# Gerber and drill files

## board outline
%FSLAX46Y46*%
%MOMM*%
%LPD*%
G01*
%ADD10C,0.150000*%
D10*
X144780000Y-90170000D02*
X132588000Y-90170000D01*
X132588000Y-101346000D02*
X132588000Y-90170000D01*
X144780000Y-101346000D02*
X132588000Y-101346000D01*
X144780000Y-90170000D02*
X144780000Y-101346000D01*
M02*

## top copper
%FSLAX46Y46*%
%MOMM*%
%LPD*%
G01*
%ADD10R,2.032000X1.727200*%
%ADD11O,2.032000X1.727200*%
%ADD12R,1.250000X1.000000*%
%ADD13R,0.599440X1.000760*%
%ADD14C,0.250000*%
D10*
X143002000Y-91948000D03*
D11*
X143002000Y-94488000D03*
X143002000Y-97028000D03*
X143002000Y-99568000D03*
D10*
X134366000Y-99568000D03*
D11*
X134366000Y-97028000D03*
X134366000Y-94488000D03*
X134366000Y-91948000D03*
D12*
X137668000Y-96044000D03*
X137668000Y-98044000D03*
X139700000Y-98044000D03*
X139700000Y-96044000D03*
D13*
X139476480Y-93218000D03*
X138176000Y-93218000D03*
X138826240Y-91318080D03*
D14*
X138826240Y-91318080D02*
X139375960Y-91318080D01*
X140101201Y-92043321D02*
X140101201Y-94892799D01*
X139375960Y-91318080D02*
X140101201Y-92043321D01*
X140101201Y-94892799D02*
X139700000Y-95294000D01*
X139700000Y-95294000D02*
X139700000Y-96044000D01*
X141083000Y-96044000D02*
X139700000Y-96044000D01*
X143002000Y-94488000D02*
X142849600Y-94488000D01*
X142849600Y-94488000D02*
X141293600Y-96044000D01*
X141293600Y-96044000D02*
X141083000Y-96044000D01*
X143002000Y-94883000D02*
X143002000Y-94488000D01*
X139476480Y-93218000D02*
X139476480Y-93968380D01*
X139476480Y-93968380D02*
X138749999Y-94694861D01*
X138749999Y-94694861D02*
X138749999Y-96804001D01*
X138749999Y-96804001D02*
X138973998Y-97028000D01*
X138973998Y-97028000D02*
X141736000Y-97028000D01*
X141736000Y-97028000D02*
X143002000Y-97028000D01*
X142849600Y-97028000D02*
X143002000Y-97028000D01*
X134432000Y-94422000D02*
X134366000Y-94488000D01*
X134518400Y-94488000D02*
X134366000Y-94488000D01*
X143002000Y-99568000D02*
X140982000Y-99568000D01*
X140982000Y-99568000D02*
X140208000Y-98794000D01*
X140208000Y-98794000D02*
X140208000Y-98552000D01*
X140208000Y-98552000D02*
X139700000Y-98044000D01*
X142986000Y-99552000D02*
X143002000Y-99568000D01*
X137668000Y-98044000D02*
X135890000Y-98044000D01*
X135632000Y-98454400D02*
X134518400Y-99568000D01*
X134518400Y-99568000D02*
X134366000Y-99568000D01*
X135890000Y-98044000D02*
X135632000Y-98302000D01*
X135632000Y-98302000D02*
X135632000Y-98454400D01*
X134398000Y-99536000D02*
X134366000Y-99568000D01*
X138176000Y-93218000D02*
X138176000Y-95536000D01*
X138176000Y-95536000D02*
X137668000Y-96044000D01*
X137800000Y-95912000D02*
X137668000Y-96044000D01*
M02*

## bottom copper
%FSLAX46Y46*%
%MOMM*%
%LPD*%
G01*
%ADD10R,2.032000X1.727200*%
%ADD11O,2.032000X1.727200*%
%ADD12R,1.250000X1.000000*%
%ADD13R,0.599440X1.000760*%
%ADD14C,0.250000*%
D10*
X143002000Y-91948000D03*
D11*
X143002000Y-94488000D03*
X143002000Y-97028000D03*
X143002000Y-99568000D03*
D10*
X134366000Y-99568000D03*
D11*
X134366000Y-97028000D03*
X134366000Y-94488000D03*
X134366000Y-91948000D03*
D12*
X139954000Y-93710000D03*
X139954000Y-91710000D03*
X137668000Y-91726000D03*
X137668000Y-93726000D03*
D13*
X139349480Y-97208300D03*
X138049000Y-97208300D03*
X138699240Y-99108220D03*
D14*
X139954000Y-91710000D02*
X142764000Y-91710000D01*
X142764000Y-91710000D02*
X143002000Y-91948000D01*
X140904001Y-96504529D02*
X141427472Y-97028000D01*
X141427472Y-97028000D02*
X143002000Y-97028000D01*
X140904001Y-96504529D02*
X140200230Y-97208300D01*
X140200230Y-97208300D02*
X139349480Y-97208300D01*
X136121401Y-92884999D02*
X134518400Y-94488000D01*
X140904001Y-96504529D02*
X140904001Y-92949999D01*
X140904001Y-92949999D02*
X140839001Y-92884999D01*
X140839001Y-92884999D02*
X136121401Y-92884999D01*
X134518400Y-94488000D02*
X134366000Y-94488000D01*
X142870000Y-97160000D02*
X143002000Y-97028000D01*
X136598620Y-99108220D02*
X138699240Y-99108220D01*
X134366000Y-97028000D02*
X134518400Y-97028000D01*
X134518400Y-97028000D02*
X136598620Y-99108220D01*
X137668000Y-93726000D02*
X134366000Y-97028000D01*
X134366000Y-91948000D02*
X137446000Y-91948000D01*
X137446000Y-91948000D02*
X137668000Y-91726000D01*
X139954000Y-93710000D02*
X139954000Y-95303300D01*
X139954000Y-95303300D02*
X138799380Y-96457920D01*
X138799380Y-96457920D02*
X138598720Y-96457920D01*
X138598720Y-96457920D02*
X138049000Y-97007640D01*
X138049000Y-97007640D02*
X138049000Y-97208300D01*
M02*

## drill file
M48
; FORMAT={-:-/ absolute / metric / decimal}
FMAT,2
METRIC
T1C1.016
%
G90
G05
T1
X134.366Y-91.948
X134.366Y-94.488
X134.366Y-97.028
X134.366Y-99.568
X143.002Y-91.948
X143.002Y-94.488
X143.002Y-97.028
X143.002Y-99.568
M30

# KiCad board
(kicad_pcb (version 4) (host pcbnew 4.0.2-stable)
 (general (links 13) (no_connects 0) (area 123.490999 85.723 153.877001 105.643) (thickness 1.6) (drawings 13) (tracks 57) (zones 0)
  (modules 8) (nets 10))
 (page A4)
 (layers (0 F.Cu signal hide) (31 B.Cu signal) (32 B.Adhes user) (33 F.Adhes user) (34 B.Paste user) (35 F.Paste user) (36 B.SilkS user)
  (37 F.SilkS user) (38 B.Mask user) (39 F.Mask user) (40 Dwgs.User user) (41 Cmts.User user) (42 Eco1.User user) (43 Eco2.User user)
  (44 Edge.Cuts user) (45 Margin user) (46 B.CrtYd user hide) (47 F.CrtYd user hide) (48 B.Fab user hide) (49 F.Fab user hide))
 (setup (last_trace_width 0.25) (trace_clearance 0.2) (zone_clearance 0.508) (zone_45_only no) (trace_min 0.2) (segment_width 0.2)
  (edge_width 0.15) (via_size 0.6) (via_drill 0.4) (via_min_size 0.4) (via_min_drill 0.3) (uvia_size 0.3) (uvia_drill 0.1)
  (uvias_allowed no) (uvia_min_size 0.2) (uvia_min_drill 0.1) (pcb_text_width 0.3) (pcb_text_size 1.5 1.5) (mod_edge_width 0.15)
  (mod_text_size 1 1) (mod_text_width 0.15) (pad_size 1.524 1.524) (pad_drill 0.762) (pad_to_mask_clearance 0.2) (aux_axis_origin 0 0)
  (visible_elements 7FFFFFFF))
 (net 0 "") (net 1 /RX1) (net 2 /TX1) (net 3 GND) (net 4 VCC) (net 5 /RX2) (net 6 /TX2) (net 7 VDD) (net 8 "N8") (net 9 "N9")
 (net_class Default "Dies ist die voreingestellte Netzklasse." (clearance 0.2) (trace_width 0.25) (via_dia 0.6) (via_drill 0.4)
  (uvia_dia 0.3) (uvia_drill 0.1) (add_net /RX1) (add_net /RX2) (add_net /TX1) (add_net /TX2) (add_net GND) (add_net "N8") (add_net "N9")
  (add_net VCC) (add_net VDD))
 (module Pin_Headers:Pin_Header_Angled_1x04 (layer F.Cu) (at 143.002 91.948)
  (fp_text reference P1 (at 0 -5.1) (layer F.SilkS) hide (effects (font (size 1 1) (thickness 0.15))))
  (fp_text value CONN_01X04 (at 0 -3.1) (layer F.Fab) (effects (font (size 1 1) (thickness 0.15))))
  (pad 1 thru_hole rect (at 0 0) (size 2.032 1.7272) (drill 1.016) (layers *.Cu *.Mask F.SilkS) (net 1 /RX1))
  (pad 2 thru_hole oval (at 0 2.54) (size 2.032 1.7272) (drill 1.016) (layers *.Cu *.Mask F.SilkS) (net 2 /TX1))
  (pad 3 thru_hole oval (at 0 5.08) (size 2.032 1.7272) (drill 1.016) (layers *.Cu *.Mask F.SilkS) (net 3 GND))
  (pad 4 thru_hole oval (at 0 7.62) (size 2.032 1.7272) (drill 1.016) (layers *.Cu *.Mask F.SilkS) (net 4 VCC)))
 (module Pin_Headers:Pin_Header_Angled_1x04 (layer F.Cu) (at 134.366 99.568 180)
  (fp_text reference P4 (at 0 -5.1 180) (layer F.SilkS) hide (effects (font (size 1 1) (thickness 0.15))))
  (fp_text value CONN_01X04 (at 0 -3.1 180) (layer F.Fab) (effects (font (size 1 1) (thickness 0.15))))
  (pad 1 thru_hole rect (at 0 0 180) (size 2.032 1.7272) (drill 1.016) (layers *.Cu *.Mask F.SilkS) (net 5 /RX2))
  (pad 2 thru_hole oval (at 0 2.54 180) (size 2.032 1.7272) (drill 1.016) (layers *.Cu *.Mask F.SilkS) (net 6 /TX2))
  (pad 3 thru_hole oval (at 0 5.08 180) (size 2.032 1.7272) (drill 1.016) (layers *.Cu *.Mask F.SilkS) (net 3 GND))
  (pad 4 thru_hole oval (at 0 7.62 180) (size 2.032 1.7272) (drill 1.016) (layers *.Cu *.Mask F.SilkS) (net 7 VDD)))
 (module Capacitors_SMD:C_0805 (layer B.Cu) (at 139.954 92.71 90)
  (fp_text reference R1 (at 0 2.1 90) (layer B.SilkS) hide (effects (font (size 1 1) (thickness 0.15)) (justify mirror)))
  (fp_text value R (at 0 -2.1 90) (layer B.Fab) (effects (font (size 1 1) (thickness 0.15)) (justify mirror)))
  (pad 1 smd rect (at -1 0 90) (size 1 1.25) (layers B.Cu B.Paste B.Mask) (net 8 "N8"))
  (pad 2 smd rect (at 1 0 90) (size 1 1.25) (layers B.Cu B.Paste B.Mask) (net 1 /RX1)))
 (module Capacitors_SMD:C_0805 (layer F.Cu) (at 137.668 97.044 270)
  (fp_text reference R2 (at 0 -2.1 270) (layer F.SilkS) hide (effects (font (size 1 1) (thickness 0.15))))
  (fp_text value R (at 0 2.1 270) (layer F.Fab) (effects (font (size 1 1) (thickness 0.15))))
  (pad 1 smd rect (at -1 0 270) (size 1 1.25) (layers F.Cu F.Paste F.Mask) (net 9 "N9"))
  (pad 2 smd rect (at 1 0 270) (size 1 1.25) (layers F.Cu F.Paste F.Mask) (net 5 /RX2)))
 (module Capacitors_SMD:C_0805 (layer B.Cu) (at 137.668 92.726 270)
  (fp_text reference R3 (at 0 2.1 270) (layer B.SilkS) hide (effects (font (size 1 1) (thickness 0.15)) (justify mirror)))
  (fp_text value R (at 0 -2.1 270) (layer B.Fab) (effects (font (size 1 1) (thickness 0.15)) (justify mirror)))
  (pad 1 smd rect (at -1 0 270) (size 1 1.25) (layers B.Cu B.Paste B.Mask) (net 7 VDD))
  (pad 2 smd rect (at 1 0 270) (size 1 1.25) (layers B.Cu B.Paste B.Mask) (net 6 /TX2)))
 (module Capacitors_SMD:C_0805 (layer F.Cu) (at 139.7 97.044 90)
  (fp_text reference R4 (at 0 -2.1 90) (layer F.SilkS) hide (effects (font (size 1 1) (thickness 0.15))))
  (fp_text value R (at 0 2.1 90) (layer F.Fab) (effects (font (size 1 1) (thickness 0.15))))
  (pad 1 smd rect (at -1 0 90) (size 1 1.25) (layers F.Cu F.Paste F.Mask) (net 4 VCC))
  (pad 2 smd rect (at 1 0 90) (size 1 1.25) (layers F.Cu F.Paste F.Mask) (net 2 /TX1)))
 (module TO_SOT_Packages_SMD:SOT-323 (layer B.Cu) (at 138.69924 98.15826 180)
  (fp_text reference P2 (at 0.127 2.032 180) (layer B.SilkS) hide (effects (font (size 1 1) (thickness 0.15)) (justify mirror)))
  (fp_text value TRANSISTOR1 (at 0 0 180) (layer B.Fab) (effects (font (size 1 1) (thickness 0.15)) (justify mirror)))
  (pad 2 smd rect (at -0.65024 0.94996 180) (size 0.59944 1.00076) (layers B.Cu B.Paste B.Mask) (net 3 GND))
  (pad 1 smd rect (at 0.65024 0.94996 180) (size 0.59944 1.00076) (layers B.Cu B.Paste B.Mask) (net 8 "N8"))
  (pad 3 smd rect (at 0 -0.94996 180) (size 0.59944 1.00076) (layers B.Cu B.Paste B.Mask) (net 6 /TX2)))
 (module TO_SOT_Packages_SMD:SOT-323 (layer F.Cu) (at 138.82624 92.26804 180)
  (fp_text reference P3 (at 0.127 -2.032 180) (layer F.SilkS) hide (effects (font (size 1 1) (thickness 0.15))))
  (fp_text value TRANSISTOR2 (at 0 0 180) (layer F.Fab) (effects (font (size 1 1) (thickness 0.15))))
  (pad 2 smd rect (at -0.65024 -0.94996 180) (size 0.59944 1.00076) (layers F.Cu F.Paste F.Mask) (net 3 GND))
  (pad 1 smd rect (at 0.65024 -0.94996 180) (size 0.59944 1.00076) (layers F.Cu F.Paste F.Mask) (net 9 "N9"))
  (pad 3 smd rect (at 0 0.94996 180) (size 0.59944 1.00076) (layers F.Cu F.Paste F.Mask) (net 2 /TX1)))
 (gr_line (start 144.78 90.17) (end 132.588 90.17) (layer Edge.Cuts) (width 0.15))
 (gr_line (start 132.588 101.346) (end 132.588 90.17) (layer Edge.Cuts) (width 0.15))
 (gr_line (start 144.78 101.346) (end 132.588 101.346) (layer Edge.Cuts) (width 0.15))
 (gr_line (start 144.78 90.17) (end 144.78 101.346) (layer Edge.Cuts) (width 0.15))
 (segment (start 144.78 90.17) (end 132.588 90.17) (width 0.25) (layer Dwgs.User) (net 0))
 (segment (start 139.954 91.71) (end 142.764 91.71) (width 0.25) (layer B.Cu) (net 1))
 (segment (start 142.764 91.71) (end 143.002 91.948) (width 0.25) (layer B.Cu) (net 1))
 (segment (start 138.82624 91.31808) (end 139.37596 91.31808) (width 0.25) (layer F.Cu) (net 2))
 (segment (start 140.101201 92.043321) (end 140.101201 94.892799) (width 0.25) (layer F.Cu) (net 2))
 (segment (start 139.37596 91.31808) (end 140.101201 92.043321) (width 0.25) (layer F.Cu) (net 2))
 (segment (start 140.101201 94.892799) (end 139.7 95.294) (width 0.25) (layer F.Cu) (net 2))
 (segment (start 139.7 95.294) (end 139.7 96.044) (width 0.25) (layer F.Cu) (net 2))
 (segment (start 141.083 96.044) (end 139.7 96.044) (width 0.25) (layer F.Cu) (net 2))
 (segment (start 143.002 94.488) (end 142.8496 94.488) (width 0.25) (layer F.Cu) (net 2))
 (segment (start 142.8496 94.488) (end 141.2936 96.044) (width 0.25) (layer F.Cu) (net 2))
 (segment (start 141.2936 96.044) (end 141.083 96.044) (width 0.25) (layer F.Cu) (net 2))
 (segment (start 143.002 94.883) (end 143.002 94.488) (width 0.25) (layer F.Cu) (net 2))
 (segment (start 140.904001 96.504529) (end 141.427472 97.028) (width 0.25) (layer B.Cu) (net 3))
 (segment (start 141.427472 97.028) (end 143.002 97.028) (width 0.25) (layer B.Cu) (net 3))
 (segment (start 140.904001 96.504529) (end 140.20023 97.2083) (width 0.25) (layer B.Cu) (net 3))
 (segment (start 140.20023 97.2083) (end 139.34948 97.2083) (width 0.25) (layer B.Cu) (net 3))
 (segment (start 139.47648 93.218) (end 139.47648 93.96838) (width 0.25) (layer F.Cu) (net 3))
 (segment (start 139.47648 93.96838) (end 138.749999 94.694861) (width 0.25) (layer F.Cu) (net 3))
 (segment (start 138.749999 94.694861) (end 138.749999 96.804001) (width 0.25) (layer F.Cu) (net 3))
 (segment (start 138.749999 96.804001) (end 138.973998 97.028) (width 0.25) (layer F.Cu) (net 3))
 (segment (start 138.973998 97.028) (end 141.736 97.028) (width 0.25) (layer F.Cu) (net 3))
 (segment (start 141.736 97.028) (end 143.002 97.028) (width 0.25) (layer F.Cu) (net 3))
 (segment (start 136.121401 92.884999) (end 134.5184 94.488) (width 0.25) (layer B.Cu) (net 3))
 (segment (start 140.904001 96.504529) (end 140.904001 92.949999) (width 0.25) (layer B.Cu) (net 3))
 (segment (start 140.904001 92.949999) (end 140.839001 92.884999) (width 0.25) (layer B.Cu) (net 3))
 (segment (start 140.839001 92.884999) (end 136.121401 92.884999) (width 0.25) (layer B.Cu) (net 3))
 (segment (start 134.5184 94.488) (end 134.366 94.488) (width 0.25) (layer B.Cu) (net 3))
 (segment (start 142.8496 97.028) (end 143.002 97.028) (width 0.25) (layer F.Cu) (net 3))
 (segment (start 134.432 94.422) (end 134.366 94.488) (width 0.25) (layer F.Cu) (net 3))
 (segment (start 142.87 97.16) (end 143.002 97.028) (width 0.25) (layer B.Cu) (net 3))
 (segment (start 134.5184 94.488) (end 134.366 94.488) (width 0.25) (layer F.Cu) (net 3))
 (segment (start 143.002 99.568) (end 140.982 99.568) (width 0.25) (layer F.Cu) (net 4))
 (segment (start 140.982 99.568) (end 140.208 98.794) (width 0.25) (layer F.Cu) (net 4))
 (segment (start 140.208 98.794) (end 140.208 98.552) (width 0.25) (layer F.Cu) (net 4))
 (segment (start 140.208 98.552) (end 139.7 98.044) (width 0.25) (layer F.Cu) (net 4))
 (segment (start 142.986 99.552) (end 143.002 99.568) (width 0.25) (layer F.Cu) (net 4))
 (segment (start 136.59862 99.10822) (end 138.69924 99.10822) (width 0.25) (layer B.Cu) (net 6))
 (segment (start 134.366 97.028) (end 134.5184 97.028) (width 0.25) (layer B.Cu) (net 6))
 (segment (start 134.5184 97.028) (end 136.59862 99.10822) (width 0.25) (layer B.Cu) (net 6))
 (segment (start 137.668 93.726) (end 134.366 97.028) (width 0.25) (layer B.Cu) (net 6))
 (segment (start 137.668 98.044) (end 135.89 98.044) (width 0.25) (layer F.Cu) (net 5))
 (segment (start 135.632 98.4544) (end 134.5184 99.568) (width 0.25) (layer F.Cu) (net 5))
 (segment (start 134.5184 99.568) (end 134.366 99.568) (width 0.25) (layer F.Cu) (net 5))
 (segment (start 135.89 98.044) (end 135.632 98.302) (width 0.25) (layer F.Cu) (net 5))
 (segment (start 135.632 98.302) (end 135.632 98.4544) (width 0.25) (layer F.Cu) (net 5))
 (segment (start 134.398 99.536) (end 134.366 99.568) (width 0.25) (layer F.Cu) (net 5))
 (segment (start 134.366 91.948) (end 137.446 91.948) (width 0.25) (layer B.Cu) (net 7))
 (segment (start 137.446 91.948) (end 137.668 91.726) (width 0.25) (layer B.Cu) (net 7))
 (segment (start 139.954 93.71) (end 139.954 95.3033) (width 0.25) (layer B.Cu) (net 8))
 (segment (start 139.954 95.3033) (end 138.79938 96.45792) (width 0.25) (layer B.Cu) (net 8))
 (segment (start 138.79938 96.45792) (end 138.59872 96.45792) (width 0.25) (layer B.Cu) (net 8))
 (segment (start 138.59872 96.45792) (end 138.049 97.00764) (width 0.25) (layer B.Cu) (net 8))
 (segment (start 138.049 97.00764) (end 138.049 97.2083) (width 0.25) (layer B.Cu) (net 8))
 (segment (start 138.176 93.218) (end 138.176 95.536) (width 0.25) (layer F.Cu) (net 9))
 (segment (start 138.176 95.536) (end 137.668 96.044) (width 0.25) (layer F.Cu) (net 9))
 (segment (start 137.8 95.912) (end 137.668 96.044) (width 0.25) (layer F.Cu) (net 9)))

